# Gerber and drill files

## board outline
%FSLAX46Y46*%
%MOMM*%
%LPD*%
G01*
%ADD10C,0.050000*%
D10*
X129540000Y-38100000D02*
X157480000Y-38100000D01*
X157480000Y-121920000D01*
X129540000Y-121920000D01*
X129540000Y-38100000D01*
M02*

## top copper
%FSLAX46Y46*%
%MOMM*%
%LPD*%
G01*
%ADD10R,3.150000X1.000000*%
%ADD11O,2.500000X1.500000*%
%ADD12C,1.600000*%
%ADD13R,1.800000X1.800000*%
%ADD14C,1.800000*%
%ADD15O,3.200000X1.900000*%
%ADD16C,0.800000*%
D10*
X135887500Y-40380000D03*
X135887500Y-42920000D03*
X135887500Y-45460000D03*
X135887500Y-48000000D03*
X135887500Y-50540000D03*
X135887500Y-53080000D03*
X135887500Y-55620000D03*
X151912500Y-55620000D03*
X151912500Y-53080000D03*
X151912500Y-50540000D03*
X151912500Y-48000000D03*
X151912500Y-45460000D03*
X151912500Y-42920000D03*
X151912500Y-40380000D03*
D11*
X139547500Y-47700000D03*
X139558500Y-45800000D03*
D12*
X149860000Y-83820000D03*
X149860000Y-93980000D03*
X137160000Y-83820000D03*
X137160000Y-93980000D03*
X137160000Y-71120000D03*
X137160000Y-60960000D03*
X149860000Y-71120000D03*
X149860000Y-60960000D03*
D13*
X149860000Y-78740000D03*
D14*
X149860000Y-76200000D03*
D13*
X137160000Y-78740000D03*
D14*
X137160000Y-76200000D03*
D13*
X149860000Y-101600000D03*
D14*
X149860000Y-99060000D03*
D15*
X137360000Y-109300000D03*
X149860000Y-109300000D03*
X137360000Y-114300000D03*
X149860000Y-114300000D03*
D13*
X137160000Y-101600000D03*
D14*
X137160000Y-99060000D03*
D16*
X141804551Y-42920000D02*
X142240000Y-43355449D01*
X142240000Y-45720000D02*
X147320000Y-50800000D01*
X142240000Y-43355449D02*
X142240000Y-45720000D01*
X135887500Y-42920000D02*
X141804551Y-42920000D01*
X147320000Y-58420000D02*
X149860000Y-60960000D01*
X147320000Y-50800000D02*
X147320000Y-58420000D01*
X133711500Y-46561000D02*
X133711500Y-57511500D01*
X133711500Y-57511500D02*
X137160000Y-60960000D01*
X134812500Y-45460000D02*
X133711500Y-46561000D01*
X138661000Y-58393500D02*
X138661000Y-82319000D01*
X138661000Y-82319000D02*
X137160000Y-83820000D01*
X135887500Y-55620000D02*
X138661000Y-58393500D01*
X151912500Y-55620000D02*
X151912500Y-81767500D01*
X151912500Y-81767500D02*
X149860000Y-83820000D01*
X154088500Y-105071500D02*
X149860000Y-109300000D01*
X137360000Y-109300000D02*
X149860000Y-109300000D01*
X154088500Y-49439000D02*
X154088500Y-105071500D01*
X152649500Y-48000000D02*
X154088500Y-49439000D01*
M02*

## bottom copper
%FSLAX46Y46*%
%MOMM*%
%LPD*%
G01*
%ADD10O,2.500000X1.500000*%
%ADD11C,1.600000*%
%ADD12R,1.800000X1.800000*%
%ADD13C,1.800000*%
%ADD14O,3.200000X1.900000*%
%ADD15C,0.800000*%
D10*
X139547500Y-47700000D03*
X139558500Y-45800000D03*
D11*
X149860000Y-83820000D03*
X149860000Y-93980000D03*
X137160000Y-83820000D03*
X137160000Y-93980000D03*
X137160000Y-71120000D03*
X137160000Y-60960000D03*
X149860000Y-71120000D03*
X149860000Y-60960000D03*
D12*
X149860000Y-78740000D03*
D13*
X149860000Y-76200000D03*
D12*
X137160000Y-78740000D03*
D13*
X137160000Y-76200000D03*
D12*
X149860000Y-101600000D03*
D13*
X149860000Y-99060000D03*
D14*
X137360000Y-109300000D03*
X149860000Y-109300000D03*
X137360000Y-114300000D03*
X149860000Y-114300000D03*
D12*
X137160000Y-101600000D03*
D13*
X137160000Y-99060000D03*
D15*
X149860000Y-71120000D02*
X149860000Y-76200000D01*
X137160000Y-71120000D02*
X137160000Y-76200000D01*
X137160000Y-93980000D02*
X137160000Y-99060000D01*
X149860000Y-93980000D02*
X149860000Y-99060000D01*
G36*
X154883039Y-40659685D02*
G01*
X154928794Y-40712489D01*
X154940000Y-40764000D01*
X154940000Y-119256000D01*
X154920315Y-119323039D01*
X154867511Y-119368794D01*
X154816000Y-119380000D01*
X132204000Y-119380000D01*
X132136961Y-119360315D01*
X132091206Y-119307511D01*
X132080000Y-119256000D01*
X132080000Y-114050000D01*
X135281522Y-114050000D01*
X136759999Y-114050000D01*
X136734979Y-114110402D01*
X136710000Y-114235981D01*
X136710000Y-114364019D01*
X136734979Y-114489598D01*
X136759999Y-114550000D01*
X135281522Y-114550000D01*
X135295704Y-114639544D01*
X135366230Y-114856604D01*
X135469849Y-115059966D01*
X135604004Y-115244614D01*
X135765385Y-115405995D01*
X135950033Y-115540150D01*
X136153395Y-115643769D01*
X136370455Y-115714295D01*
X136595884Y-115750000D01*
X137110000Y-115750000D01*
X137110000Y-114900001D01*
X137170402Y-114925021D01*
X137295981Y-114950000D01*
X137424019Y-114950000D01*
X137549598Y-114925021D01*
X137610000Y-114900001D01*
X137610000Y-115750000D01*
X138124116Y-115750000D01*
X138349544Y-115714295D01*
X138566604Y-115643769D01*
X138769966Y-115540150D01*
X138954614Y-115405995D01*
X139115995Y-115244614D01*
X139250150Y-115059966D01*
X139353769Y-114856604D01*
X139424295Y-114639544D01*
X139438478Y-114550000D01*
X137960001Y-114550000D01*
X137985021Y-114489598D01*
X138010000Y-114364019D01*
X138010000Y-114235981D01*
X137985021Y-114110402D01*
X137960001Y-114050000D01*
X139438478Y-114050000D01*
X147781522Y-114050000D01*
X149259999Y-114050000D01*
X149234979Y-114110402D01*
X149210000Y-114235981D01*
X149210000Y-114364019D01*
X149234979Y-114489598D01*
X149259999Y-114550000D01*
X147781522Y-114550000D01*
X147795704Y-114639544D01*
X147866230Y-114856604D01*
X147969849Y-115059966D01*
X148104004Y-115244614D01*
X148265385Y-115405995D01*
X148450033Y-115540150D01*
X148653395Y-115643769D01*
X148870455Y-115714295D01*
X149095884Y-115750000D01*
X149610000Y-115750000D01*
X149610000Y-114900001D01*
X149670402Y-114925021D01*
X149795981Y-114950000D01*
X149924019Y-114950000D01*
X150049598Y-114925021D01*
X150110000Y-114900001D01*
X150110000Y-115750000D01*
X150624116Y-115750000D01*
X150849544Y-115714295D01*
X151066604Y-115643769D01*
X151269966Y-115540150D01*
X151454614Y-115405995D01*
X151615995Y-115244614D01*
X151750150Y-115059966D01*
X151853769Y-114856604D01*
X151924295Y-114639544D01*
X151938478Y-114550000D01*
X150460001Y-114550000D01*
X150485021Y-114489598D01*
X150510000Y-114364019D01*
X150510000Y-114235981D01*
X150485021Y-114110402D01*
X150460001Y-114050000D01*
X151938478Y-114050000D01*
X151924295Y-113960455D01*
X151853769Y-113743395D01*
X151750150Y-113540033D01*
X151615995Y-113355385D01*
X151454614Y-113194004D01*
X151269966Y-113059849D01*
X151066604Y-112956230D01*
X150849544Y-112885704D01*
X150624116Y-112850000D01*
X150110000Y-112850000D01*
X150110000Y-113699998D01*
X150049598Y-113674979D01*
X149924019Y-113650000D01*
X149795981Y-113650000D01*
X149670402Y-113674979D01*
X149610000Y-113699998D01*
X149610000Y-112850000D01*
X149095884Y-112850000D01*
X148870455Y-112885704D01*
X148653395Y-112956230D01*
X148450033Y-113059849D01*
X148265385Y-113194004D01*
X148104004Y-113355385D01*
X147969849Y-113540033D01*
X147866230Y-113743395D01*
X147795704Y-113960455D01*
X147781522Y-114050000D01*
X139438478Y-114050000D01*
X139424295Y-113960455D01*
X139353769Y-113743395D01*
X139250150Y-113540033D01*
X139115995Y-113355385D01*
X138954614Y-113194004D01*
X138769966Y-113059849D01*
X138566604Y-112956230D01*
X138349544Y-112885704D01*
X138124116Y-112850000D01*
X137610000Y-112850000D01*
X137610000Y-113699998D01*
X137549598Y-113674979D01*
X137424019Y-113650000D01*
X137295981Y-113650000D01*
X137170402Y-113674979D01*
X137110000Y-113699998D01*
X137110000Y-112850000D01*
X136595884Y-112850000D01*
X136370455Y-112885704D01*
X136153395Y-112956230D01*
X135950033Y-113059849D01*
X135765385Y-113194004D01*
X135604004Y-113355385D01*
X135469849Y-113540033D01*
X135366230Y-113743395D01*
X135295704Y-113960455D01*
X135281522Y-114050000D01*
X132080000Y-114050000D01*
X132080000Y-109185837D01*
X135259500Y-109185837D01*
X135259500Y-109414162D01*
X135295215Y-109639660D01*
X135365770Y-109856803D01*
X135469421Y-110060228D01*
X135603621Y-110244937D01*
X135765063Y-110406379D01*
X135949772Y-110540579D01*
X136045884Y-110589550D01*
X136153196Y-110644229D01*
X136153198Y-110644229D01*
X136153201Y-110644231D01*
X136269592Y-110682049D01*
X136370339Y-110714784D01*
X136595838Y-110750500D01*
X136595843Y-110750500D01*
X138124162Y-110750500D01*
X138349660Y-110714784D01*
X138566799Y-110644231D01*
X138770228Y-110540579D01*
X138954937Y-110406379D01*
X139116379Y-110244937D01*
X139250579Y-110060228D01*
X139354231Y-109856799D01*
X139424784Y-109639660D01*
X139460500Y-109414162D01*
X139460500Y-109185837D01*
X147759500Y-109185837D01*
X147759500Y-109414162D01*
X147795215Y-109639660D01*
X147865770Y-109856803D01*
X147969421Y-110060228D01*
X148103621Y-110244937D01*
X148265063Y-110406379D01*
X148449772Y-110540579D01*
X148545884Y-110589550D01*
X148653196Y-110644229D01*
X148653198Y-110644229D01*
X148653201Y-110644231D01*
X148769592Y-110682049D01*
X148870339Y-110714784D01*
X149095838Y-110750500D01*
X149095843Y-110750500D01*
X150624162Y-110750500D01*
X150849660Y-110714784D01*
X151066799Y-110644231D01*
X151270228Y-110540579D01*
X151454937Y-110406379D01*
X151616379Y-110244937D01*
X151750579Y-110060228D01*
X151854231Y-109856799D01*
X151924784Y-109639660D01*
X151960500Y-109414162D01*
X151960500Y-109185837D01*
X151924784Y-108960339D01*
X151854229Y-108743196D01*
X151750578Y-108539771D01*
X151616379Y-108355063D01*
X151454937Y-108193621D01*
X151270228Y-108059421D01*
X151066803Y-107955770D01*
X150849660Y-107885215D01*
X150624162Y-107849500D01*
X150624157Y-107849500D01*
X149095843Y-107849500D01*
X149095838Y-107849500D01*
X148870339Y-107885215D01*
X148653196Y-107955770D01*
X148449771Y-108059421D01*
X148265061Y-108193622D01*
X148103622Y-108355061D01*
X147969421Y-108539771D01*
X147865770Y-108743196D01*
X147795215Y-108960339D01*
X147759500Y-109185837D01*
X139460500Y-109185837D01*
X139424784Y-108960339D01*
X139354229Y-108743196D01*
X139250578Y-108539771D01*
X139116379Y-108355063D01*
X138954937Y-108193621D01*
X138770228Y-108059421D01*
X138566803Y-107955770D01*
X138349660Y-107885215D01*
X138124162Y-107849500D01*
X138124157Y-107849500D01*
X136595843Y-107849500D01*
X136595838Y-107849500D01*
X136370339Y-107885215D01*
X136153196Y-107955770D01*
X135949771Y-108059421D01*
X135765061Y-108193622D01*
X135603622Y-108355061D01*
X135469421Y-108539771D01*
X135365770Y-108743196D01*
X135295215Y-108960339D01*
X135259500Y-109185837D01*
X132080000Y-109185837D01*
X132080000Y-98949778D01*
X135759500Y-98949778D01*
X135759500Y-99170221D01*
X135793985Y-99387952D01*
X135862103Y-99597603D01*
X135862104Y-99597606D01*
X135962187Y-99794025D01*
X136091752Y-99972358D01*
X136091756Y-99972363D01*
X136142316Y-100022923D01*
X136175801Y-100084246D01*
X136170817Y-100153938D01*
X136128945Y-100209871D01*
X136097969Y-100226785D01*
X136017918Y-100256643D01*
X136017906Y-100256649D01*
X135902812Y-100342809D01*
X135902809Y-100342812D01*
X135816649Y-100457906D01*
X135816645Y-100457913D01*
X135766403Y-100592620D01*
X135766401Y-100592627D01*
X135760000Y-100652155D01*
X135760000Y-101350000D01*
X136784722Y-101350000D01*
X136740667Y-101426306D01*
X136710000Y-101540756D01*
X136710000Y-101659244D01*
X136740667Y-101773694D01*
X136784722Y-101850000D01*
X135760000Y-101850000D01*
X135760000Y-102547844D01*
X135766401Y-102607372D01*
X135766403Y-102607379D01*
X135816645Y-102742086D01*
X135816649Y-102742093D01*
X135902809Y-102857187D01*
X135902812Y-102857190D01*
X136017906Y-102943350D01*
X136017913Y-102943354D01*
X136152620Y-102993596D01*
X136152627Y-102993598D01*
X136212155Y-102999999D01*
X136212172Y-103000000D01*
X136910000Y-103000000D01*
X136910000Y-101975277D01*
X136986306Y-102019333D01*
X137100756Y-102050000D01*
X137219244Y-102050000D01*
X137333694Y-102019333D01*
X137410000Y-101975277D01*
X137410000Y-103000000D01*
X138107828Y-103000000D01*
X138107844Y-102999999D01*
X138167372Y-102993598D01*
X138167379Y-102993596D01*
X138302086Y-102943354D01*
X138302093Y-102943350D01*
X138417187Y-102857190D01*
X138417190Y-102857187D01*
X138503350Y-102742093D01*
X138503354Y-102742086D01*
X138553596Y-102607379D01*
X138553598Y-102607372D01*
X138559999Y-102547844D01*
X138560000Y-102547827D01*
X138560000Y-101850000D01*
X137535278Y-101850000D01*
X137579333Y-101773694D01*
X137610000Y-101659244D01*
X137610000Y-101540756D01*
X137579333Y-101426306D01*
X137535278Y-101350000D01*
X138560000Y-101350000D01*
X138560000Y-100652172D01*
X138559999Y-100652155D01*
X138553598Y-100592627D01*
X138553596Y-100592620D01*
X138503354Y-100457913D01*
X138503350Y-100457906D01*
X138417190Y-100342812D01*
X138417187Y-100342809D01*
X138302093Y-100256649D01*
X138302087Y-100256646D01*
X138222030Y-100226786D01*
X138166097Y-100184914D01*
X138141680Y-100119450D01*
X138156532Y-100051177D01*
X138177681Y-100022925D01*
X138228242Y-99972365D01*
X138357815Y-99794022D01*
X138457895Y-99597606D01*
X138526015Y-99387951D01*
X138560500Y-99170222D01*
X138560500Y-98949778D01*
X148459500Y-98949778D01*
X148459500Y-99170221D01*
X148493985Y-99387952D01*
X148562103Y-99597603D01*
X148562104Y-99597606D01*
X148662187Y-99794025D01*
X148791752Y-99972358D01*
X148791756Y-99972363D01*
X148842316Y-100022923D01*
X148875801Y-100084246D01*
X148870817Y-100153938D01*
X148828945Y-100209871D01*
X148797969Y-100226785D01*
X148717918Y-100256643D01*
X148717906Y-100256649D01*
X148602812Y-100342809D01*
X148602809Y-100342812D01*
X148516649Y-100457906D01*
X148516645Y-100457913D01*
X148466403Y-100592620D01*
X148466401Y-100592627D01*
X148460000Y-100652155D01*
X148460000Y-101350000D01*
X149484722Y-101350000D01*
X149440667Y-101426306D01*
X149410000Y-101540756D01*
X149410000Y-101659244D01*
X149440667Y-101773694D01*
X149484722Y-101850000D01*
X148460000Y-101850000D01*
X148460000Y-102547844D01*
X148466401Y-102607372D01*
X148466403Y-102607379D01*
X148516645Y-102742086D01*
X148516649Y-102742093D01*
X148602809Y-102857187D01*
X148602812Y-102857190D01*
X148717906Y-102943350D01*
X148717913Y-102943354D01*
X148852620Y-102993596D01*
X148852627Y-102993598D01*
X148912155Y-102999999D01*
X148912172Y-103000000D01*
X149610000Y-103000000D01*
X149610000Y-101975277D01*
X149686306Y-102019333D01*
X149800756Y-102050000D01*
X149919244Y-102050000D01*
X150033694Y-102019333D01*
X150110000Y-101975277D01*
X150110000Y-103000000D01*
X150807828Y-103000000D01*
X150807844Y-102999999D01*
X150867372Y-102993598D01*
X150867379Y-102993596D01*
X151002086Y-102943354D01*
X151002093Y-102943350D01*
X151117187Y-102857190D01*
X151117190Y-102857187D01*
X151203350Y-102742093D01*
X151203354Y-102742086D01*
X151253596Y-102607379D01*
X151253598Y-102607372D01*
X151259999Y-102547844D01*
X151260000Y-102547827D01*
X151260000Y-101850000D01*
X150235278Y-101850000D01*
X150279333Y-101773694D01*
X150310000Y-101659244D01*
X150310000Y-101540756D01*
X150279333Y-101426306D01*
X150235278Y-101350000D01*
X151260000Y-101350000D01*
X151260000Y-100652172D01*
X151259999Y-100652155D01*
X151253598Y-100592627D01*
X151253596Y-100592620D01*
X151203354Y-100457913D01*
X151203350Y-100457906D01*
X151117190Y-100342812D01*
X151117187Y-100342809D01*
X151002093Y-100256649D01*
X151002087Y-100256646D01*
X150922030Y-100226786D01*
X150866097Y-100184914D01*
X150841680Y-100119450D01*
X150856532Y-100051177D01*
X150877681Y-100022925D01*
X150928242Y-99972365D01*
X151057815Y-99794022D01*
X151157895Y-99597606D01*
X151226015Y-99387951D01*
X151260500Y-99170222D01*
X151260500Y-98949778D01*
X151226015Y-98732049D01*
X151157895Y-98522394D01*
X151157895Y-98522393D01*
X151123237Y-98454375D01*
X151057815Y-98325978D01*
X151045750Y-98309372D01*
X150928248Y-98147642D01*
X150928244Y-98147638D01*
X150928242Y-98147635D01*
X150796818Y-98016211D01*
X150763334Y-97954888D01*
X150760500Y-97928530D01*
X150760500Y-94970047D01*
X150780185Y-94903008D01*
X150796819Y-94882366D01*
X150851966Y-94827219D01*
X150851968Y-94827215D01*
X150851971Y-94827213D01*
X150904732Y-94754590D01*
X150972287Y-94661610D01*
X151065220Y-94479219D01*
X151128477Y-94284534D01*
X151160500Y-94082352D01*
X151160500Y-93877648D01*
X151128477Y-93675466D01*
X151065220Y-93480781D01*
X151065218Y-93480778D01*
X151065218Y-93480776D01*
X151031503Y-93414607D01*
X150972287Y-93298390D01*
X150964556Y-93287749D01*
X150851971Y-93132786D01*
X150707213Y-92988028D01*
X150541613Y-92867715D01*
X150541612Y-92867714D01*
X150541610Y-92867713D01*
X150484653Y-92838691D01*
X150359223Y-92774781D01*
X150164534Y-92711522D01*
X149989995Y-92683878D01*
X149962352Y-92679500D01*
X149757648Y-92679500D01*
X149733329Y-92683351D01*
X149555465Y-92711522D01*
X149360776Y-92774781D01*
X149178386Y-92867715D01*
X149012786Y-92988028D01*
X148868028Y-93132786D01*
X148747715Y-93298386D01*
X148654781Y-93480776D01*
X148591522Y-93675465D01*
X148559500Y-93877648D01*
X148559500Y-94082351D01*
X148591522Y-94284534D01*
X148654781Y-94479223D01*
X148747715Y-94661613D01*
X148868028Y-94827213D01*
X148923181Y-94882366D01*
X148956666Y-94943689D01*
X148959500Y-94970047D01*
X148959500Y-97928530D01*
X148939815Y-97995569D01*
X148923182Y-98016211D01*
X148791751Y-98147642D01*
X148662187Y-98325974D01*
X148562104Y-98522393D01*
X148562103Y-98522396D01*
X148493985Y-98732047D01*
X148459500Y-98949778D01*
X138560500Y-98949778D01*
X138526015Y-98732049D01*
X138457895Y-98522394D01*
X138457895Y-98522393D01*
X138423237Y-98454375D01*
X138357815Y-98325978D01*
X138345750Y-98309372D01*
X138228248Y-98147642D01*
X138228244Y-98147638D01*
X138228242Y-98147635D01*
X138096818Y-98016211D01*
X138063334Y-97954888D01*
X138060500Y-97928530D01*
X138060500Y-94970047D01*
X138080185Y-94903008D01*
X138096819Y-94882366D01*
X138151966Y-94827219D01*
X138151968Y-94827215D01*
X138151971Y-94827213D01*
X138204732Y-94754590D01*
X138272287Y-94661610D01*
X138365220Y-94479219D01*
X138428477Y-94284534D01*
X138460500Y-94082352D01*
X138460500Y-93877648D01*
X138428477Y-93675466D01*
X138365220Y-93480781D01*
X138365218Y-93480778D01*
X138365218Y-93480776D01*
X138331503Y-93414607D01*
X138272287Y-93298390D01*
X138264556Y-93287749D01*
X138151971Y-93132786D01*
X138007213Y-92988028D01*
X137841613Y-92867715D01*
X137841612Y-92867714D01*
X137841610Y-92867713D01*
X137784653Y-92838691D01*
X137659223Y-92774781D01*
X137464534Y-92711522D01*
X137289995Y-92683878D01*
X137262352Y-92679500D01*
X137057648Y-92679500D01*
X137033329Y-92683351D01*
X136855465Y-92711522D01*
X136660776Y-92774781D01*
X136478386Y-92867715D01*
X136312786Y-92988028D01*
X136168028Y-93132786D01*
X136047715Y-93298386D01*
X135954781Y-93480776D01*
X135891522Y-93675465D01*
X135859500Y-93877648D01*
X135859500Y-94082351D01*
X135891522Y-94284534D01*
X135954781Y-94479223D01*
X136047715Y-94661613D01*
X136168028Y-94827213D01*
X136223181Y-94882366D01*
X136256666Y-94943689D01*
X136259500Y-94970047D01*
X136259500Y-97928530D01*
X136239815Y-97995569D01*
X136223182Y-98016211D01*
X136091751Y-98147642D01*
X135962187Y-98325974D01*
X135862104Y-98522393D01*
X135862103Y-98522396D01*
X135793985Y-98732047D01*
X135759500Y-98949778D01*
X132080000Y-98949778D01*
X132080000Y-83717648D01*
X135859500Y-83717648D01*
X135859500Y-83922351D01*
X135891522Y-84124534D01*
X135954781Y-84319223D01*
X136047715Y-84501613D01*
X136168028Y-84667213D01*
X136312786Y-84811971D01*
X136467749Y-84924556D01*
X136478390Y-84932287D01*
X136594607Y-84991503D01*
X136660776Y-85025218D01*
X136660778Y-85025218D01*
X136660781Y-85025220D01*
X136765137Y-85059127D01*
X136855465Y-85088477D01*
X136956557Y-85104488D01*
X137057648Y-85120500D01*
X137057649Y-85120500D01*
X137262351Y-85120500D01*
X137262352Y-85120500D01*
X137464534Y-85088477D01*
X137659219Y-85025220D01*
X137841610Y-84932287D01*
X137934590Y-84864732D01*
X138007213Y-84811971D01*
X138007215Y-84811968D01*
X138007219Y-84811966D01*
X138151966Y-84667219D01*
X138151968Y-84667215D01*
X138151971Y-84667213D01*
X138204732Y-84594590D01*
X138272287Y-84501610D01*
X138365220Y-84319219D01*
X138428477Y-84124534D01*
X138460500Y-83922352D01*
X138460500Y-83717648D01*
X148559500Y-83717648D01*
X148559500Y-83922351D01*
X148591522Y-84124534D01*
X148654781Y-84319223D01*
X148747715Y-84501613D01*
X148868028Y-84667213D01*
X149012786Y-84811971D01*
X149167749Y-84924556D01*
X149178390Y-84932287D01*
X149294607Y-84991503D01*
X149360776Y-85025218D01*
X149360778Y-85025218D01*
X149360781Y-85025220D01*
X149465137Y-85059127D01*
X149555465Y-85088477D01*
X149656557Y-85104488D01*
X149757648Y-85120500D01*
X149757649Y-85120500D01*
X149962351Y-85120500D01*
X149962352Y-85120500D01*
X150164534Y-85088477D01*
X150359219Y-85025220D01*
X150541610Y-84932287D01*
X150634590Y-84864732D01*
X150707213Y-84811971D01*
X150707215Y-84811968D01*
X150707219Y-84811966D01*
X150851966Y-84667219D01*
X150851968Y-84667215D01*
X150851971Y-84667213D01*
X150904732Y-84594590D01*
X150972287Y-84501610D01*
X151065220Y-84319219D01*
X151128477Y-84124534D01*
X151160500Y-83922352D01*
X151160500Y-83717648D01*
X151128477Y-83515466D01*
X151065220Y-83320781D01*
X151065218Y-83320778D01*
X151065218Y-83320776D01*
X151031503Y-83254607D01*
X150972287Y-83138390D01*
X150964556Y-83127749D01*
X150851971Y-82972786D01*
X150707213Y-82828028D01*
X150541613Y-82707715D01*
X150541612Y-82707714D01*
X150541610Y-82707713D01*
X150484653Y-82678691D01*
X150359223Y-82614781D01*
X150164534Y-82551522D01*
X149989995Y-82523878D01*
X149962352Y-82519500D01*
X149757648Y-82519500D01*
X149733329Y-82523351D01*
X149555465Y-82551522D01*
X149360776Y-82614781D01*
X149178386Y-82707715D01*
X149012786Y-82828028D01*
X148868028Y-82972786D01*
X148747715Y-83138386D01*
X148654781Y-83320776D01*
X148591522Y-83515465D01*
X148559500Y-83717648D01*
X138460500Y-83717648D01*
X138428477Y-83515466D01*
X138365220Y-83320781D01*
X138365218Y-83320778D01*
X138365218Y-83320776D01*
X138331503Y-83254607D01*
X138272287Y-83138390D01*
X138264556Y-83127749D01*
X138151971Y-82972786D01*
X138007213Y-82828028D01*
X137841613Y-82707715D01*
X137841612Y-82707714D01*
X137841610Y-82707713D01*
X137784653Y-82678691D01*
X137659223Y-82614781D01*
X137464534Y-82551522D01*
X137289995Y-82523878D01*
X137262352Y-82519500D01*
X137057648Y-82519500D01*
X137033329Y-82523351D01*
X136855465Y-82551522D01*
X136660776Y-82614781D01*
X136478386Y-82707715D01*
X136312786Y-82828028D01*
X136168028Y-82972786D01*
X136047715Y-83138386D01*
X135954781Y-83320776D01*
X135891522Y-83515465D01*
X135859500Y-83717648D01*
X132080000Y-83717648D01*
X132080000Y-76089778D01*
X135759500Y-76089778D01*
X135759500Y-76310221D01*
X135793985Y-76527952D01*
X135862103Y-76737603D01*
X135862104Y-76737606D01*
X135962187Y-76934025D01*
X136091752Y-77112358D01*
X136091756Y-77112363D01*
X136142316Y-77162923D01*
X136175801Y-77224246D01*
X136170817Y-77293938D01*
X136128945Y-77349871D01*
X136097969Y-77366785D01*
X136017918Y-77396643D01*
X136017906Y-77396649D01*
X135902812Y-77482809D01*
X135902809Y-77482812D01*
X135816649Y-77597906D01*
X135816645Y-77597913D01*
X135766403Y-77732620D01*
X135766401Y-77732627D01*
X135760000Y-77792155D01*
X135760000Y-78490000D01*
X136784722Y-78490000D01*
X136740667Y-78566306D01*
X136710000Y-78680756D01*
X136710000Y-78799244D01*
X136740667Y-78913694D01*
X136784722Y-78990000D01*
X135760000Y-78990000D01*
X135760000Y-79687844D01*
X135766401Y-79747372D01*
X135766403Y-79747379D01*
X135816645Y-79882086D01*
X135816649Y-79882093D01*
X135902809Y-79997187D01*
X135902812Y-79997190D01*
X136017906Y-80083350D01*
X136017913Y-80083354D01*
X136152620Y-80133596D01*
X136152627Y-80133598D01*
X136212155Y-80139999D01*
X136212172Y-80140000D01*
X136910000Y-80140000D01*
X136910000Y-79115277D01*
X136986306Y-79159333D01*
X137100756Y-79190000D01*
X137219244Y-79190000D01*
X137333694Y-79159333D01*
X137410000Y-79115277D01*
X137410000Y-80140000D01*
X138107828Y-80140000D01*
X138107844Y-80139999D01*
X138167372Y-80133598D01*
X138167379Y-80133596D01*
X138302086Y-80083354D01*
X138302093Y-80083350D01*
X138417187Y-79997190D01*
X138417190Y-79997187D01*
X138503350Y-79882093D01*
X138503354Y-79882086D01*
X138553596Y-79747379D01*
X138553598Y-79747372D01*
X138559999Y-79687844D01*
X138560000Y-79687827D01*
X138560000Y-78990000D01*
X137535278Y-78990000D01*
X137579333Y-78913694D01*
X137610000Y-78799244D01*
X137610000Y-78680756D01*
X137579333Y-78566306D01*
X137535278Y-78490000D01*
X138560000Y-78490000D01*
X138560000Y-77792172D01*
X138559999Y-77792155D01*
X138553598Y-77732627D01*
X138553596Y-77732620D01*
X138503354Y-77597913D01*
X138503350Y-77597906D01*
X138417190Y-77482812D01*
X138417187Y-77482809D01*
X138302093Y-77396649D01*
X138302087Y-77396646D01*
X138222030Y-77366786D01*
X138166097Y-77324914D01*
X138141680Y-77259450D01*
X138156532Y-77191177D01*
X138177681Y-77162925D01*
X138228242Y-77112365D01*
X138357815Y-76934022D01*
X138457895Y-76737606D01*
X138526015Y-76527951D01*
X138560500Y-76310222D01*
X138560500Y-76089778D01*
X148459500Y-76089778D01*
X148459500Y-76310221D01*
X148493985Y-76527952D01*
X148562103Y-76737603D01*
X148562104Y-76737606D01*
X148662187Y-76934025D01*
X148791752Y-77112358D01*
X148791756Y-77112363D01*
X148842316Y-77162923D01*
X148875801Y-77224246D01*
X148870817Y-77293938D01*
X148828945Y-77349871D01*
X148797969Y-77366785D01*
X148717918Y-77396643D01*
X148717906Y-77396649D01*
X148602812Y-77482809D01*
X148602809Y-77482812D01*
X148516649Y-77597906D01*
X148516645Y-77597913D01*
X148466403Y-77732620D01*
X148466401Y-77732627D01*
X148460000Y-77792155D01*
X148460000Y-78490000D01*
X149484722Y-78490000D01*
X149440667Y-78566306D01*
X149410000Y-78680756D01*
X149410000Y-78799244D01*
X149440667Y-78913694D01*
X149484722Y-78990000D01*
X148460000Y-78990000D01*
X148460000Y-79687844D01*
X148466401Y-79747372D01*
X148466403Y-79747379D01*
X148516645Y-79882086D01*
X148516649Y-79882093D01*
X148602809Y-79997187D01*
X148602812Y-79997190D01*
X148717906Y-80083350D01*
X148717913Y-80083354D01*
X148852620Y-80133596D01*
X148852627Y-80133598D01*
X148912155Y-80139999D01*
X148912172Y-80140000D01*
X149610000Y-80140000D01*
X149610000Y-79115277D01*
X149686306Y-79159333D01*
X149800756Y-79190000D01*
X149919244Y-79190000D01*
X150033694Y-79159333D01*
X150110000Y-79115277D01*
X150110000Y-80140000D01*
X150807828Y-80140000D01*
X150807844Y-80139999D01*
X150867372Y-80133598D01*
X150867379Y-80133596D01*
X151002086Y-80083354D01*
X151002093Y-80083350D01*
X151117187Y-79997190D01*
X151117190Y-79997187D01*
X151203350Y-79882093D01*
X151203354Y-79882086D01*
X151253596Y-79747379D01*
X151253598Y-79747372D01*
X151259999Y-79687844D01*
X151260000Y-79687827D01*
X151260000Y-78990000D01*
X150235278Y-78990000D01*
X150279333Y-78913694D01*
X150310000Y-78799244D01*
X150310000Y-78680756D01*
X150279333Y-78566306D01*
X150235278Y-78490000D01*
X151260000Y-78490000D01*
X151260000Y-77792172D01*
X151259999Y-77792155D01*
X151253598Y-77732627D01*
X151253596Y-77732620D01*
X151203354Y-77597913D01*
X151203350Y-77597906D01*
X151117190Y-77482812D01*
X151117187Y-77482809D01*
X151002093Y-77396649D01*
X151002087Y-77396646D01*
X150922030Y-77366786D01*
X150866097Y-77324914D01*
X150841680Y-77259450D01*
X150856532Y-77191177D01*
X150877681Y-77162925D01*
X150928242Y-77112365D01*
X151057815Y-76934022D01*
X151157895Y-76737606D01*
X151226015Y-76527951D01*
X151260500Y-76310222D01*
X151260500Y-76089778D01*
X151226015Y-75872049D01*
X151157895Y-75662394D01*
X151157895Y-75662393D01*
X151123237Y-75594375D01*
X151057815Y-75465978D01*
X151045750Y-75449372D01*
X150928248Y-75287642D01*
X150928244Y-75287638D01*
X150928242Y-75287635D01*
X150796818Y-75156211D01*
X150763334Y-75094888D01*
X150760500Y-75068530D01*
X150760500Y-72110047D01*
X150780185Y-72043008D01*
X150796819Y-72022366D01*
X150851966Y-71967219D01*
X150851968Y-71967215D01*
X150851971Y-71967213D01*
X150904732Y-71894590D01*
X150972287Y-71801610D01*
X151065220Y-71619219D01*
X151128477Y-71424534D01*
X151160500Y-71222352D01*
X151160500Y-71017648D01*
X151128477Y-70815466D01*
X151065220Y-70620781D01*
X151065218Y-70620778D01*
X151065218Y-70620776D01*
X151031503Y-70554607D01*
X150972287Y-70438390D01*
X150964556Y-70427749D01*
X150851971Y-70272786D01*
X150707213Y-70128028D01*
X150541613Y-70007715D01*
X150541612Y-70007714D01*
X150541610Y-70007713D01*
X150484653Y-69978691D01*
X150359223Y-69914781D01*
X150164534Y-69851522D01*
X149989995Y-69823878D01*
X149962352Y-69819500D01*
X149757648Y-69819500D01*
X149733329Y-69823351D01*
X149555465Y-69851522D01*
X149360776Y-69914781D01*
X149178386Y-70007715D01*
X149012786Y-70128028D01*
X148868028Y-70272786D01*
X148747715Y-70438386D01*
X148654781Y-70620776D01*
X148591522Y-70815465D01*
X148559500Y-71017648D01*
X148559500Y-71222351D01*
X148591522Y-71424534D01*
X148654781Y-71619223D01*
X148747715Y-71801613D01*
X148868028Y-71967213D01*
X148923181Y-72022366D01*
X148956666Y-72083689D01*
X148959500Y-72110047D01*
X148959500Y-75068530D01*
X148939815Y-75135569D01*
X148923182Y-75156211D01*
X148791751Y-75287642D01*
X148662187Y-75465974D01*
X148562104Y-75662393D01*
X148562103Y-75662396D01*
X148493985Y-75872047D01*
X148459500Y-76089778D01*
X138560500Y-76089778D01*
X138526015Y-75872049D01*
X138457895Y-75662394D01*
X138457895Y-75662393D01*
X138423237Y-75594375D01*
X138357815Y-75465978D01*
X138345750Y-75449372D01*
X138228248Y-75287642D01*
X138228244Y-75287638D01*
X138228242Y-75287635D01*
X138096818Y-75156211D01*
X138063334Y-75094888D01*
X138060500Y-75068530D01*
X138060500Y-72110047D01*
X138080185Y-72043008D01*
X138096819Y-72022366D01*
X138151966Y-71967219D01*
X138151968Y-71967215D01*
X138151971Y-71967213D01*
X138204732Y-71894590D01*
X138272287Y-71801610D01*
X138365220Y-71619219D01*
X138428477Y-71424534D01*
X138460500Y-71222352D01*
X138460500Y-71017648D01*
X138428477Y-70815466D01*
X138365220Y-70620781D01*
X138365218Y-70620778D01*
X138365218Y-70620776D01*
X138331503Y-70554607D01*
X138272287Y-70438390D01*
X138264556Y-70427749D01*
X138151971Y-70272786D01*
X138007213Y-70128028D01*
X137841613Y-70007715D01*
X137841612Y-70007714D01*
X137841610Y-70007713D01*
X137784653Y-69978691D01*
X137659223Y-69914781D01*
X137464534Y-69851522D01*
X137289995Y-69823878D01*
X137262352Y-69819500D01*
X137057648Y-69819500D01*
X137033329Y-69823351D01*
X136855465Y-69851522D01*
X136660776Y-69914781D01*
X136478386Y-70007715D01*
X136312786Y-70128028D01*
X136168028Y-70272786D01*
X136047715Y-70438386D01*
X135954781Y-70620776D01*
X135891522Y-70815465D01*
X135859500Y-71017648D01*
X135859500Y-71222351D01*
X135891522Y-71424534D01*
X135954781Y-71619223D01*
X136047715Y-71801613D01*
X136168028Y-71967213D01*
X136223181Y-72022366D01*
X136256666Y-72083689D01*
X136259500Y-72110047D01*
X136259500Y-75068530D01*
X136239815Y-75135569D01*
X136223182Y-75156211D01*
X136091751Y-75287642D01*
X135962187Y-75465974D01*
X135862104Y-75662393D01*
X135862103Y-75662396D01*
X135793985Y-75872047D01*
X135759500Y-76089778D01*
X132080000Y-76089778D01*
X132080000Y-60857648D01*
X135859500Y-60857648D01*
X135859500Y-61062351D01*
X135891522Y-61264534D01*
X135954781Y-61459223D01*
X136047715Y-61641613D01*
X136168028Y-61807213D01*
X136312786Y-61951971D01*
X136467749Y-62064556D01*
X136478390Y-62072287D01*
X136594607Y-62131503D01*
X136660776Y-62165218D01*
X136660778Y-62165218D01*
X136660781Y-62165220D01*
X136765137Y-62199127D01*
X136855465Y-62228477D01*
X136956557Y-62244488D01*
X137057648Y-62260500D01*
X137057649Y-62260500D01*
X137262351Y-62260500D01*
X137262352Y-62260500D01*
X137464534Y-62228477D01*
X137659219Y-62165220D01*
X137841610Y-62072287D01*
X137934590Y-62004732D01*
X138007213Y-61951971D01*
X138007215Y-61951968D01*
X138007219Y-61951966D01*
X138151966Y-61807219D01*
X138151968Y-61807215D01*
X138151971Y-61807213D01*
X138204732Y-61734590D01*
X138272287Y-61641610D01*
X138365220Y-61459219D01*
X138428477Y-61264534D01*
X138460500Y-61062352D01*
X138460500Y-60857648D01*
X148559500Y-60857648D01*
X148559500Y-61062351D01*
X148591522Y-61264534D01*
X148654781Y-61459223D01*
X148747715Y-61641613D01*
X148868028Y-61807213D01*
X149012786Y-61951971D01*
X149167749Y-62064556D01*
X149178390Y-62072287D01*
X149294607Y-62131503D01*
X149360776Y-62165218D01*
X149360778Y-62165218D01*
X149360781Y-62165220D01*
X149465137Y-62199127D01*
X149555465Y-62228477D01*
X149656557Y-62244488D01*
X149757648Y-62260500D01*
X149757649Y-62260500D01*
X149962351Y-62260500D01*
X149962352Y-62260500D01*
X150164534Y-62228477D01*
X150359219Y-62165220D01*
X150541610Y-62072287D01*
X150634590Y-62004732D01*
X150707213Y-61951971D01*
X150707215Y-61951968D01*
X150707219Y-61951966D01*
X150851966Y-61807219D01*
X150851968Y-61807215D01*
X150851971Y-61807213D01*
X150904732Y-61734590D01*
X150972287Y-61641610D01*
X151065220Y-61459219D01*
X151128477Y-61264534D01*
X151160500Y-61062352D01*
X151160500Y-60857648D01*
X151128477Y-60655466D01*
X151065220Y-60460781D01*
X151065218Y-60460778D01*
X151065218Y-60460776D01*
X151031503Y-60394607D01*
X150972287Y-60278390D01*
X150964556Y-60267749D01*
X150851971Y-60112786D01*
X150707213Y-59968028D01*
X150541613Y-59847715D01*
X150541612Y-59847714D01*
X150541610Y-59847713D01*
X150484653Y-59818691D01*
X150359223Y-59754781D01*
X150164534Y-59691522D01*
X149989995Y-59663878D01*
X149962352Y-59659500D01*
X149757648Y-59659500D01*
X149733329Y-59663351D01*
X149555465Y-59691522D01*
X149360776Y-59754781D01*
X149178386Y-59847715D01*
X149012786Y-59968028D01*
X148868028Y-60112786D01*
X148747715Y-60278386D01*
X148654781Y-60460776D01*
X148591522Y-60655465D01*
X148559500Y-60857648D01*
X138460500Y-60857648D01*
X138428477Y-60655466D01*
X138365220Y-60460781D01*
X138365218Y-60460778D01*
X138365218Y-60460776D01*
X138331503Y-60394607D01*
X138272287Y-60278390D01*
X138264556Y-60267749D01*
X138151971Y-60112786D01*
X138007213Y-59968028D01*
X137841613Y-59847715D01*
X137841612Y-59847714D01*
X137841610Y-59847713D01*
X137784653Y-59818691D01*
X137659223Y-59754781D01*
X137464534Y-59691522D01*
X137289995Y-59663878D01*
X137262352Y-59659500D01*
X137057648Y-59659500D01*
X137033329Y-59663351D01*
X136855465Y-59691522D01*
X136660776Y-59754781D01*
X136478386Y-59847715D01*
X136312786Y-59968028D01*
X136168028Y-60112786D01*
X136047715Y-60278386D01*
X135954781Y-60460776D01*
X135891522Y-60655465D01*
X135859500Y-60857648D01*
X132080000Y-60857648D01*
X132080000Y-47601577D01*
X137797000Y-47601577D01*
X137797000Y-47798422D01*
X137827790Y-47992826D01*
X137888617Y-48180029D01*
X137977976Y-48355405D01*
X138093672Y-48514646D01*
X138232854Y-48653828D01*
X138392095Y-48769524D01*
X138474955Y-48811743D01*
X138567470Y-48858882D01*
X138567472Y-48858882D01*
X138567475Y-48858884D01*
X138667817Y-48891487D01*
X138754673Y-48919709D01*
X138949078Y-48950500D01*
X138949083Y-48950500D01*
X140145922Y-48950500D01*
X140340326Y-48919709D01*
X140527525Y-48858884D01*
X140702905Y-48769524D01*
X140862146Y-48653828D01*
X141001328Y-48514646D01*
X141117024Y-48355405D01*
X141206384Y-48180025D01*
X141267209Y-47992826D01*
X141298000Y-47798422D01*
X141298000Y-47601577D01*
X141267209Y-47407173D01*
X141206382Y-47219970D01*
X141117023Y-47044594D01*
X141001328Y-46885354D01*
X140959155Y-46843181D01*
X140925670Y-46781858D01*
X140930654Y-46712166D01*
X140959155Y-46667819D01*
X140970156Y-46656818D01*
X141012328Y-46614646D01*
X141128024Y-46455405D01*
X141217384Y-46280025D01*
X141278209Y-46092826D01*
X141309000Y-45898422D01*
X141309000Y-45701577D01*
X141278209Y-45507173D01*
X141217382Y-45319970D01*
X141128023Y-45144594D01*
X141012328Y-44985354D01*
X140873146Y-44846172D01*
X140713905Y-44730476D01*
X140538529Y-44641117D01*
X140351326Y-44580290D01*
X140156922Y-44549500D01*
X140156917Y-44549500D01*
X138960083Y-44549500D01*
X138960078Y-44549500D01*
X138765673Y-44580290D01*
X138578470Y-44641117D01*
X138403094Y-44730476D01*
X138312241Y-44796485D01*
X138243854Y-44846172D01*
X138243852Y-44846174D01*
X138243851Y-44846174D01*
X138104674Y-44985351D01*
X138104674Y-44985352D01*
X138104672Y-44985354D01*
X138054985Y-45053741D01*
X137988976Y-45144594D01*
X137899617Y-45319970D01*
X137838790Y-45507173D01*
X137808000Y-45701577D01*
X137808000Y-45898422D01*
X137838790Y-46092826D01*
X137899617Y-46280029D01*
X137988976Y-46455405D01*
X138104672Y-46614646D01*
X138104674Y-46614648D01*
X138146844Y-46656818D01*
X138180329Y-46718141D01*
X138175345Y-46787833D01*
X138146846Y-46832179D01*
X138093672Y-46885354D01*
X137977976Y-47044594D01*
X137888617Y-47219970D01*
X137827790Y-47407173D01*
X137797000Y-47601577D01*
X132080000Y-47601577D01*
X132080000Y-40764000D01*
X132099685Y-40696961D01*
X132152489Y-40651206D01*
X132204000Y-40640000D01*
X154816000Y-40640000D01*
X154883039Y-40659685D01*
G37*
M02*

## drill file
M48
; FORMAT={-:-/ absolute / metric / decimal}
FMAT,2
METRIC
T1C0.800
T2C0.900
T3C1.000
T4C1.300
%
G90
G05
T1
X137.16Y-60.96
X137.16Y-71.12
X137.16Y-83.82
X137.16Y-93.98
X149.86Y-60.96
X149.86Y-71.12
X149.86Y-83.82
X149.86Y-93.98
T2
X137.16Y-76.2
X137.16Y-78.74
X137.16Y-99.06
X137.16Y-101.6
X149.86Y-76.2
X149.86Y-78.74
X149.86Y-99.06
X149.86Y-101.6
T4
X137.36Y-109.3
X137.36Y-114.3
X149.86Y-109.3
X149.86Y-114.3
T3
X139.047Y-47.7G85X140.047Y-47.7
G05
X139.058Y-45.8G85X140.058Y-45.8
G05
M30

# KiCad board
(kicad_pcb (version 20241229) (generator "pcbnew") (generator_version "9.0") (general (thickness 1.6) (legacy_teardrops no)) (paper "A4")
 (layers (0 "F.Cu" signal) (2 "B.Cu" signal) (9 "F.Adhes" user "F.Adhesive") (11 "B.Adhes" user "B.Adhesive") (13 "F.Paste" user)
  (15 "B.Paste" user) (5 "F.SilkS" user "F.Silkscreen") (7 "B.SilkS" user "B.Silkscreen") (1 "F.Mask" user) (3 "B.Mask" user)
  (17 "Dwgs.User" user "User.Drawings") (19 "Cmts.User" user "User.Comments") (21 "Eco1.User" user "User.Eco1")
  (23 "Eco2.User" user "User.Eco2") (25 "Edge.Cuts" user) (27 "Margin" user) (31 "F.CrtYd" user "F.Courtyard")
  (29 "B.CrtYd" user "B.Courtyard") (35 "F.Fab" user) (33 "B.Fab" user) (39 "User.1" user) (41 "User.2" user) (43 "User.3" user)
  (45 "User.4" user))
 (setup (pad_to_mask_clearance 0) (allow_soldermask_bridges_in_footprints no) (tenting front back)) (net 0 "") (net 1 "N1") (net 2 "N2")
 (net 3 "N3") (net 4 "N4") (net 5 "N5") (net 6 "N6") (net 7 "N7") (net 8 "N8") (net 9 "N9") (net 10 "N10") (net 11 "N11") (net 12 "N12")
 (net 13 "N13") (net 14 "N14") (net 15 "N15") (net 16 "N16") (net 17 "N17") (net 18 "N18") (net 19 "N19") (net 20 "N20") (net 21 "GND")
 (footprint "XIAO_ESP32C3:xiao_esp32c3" (layer "F.Cu") (at 144.4875 49.8)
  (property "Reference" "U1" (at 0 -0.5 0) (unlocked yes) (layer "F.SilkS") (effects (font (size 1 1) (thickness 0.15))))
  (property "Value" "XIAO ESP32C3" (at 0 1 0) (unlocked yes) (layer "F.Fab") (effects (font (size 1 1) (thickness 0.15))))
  (pad "1" smd rect (at -8.6 -9.42) (size 3.15 1) (layers "F.Cu" "F.Mask" "F.Paste") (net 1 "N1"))
  (pad "2" smd rect (at -8.6 -6.88) (size 3.15 1) (layers "F.Cu" "F.Mask" "F.Paste") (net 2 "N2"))
  (pad "3" smd rect (at -8.6 -4.34) (size 3.15 1) (layers "F.Cu" "F.Mask" "F.Paste") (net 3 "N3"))
  (pad "4" smd rect (at -8.6 -1.8) (size 3.15 1) (layers "F.Cu" "F.Mask" "F.Paste") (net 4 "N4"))
  (pad "5" smd rect (at -8.6 0.74) (size 3.15 1) (layers "F.Cu" "F.Mask" "F.Paste") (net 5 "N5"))
  (pad "6" smd rect (at -8.6 3.28) (size 3.15 1) (layers "F.Cu" "F.Mask" "F.Paste") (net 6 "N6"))
  (pad "7" smd rect (at -8.6 5.82) (size 3.15 1) (layers "F.Cu" "F.Mask" "F.Paste") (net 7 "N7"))
  (pad "8" smd rect (at 7.425 5.82) (size 3.15 1) (layers "F.Cu" "F.Mask" "F.Paste") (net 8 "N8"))
  (pad "9" smd rect (at 7.425 3.28) (size 3.15 1) (layers "F.Cu" "F.Mask" "F.Paste") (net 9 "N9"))
  (pad "10" smd rect (at 7.425 0.74) (size 3.15 1) (layers "F.Cu" "F.Mask" "F.Paste") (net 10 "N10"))
  (pad "11" smd rect (at 7.425 -1.8) (size 3.15 1) (layers "F.Cu" "F.Mask" "F.Paste") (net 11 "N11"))
  (pad "12" smd rect (at 7.425 -4.34) (size 3.15 1) (layers "F.Cu" "F.Mask" "F.Paste") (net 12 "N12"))
  (pad "13" smd rect (at 7.425 -6.88) (size 3.15 1) (layers "F.Cu" "F.Mask" "F.Paste") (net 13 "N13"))
  (pad "14" smd rect (at 7.425 -9.42) (size 3.15 1) (layers "F.Cu" "F.Mask" "F.Paste") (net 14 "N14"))
  (pad "B+" thru_hole oval (at -4.94 -2.1) (size 2.5 1.5) (drill oval 2 1) (layers "*.Cu" "*.Mask") (remove_unused_layers no) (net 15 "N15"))
  (pad "B-" thru_hole oval (at -4.929 -4) (size 2.5 1.5) (drill oval 2 1) (layers "*.Cu" "*.Mask") (remove_unused_layers no) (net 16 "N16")))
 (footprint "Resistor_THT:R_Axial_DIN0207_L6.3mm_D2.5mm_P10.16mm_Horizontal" (layer "F.Cu") (at 149.86 83.82 -90)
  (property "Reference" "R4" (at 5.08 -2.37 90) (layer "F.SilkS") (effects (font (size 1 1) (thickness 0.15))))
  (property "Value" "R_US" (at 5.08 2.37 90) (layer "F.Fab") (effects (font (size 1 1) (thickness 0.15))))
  (pad "1" thru_hole circle (at 0 0 270) (size 1.6 1.6) (drill 0.8) (layers "*.Cu" "*.Mask") (remove_unused_layers no) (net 8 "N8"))
  (pad "2" thru_hole circle (at 10.16 0 270) (size 1.6 1.6) (drill 0.8) (layers "*.Cu" "*.Mask") (remove_unused_layers no) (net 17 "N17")))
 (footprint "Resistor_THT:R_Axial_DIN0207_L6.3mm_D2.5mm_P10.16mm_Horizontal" (layer "F.Cu") (at 137.16 83.82 -90)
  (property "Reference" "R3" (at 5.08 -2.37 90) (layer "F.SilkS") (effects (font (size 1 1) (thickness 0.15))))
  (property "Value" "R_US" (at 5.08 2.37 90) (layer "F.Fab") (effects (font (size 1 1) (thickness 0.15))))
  (pad "1" thru_hole circle (at 0 0 270) (size 1.6 1.6) (drill 0.8) (layers "*.Cu" "*.Mask") (remove_unused_layers no) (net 7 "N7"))
  (pad "2" thru_hole circle (at 10.16 0 270) (size 1.6 1.6) (drill 0.8) (layers "*.Cu" "*.Mask") (remove_unused_layers no) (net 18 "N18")))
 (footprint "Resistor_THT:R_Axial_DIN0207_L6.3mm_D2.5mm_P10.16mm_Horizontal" (layer "F.Cu") (at 137.16 71.12 90)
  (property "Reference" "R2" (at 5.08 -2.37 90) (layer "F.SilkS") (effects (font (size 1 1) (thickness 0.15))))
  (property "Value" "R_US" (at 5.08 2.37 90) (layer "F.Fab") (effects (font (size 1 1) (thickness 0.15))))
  (pad "1" thru_hole circle (at 0 0 90) (size 1.6 1.6) (drill 0.8) (layers "*.Cu" "*.Mask") (remove_unused_layers no) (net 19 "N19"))
  (pad "2" thru_hole circle (at 10.16 0 90) (size 1.6 1.6) (drill 0.8) (layers "*.Cu" "*.Mask") (remove_unused_layers no) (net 3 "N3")))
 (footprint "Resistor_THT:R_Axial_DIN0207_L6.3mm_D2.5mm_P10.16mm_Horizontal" (layer "F.Cu") (at 149.86 71.12 90)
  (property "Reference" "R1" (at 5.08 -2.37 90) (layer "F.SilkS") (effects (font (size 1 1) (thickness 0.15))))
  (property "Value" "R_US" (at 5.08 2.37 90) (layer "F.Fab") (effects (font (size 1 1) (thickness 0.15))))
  (pad "1" thru_hole circle (at 0 0 90) (size 1.6 1.6) (drill 0.8) (layers "*.Cu" "*.Mask") (remove_unused_layers no) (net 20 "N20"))
  (pad "2" thru_hole circle (at 10.16 0 90) (size 1.6 1.6) (drill 0.8) (layers "*.Cu" "*.Mask") (remove_unused_layers no) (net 2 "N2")))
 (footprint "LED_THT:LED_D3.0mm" (layer "F.Cu") (at 149.86 78.74 90)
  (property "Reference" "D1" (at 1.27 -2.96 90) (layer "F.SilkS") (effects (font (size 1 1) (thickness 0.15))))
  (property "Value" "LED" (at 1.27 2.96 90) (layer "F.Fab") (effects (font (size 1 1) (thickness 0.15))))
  (pad "1" thru_hole rect (at 0 0 90) (size 1.8 1.8) (drill 0.9) (layers "*.Cu" "*.Mask") (remove_unused_layers no) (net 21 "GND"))
  (pad "2" thru_hole circle (at 2.54 0 90) (size 1.8 1.8) (drill 0.9) (layers "*.Cu" "*.Mask") (remove_unused_layers no) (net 20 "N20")))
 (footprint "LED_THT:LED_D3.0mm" (layer "F.Cu") (at 137.16 78.74 90)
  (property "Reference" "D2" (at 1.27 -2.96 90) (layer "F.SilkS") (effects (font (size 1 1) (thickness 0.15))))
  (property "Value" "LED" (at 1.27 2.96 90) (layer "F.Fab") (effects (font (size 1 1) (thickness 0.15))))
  (pad "1" thru_hole rect (at 0 0 90) (size 1.8 1.8) (drill 0.9) (layers "*.Cu" "*.Mask") (remove_unused_layers no) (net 21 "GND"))
  (pad "2" thru_hole circle (at 2.54 0 90) (size 1.8 1.8) (drill 0.9) (layers "*.Cu" "*.Mask") (remove_unused_layers no) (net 19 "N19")))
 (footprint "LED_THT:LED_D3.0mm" (layer "F.Cu") (at 149.86 101.6 90)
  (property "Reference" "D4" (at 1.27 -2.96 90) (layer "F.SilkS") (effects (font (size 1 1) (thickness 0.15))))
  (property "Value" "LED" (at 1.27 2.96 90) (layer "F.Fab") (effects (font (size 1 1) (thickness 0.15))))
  (pad "1" thru_hole rect (at 0 0 90) (size 1.8 1.8) (drill 0.9) (layers "*.Cu" "*.Mask") (remove_unused_layers no) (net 21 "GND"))
  (pad "2" thru_hole circle (at 2.54 0 90) (size 1.8 1.8) (drill 0.9) (layers "*.Cu" "*.Mask") (remove_unused_layers no) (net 17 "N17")))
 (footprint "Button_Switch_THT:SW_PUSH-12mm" (layer "F.Cu") (at 137.36 109.3)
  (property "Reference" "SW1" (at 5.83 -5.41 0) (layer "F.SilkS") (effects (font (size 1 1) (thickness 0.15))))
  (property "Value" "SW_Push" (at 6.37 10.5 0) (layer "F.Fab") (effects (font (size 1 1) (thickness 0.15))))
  (pad "1" thru_hole oval (at 0 0) (size 3.2 1.9) (drill 1.3) (layers "*.Cu" "*.Mask") (remove_unused_layers no) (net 11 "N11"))
  (pad "1" thru_hole oval (at 12.5 0) (size 3.2 1.9) (drill 1.3) (layers "*.Cu" "*.Mask") (remove_unused_layers no) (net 11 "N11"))
  (pad "2" thru_hole oval (at 0 5) (size 3.2 1.9) (drill 1.3) (layers "*.Cu" "*.Mask") (remove_unused_layers no) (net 21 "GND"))
  (pad "2" thru_hole oval (at 12.5 5) (size 3.2 1.9) (drill 1.3) (layers "*.Cu" "*.Mask") (remove_unused_layers no) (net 21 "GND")))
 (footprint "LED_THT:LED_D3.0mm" (layer "F.Cu") (at 137.16 101.6 90)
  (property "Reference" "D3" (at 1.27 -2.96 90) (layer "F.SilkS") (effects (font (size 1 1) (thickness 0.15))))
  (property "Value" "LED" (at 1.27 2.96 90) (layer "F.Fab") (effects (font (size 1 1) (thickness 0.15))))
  (pad "1" thru_hole rect (at 0 0 90) (size 1.8 1.8) (drill 0.9) (layers "*.Cu" "*.Mask") (remove_unused_layers no) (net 21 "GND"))
  (pad "2" thru_hole circle (at 2.54 0 90) (size 1.8 1.8) (drill 0.9) (layers "*.Cu" "*.Mask") (remove_unused_layers no) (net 18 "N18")))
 (gr_rect (start 129.54 38.1) (end 157.48 121.92) (stroke (width 0.05) (type default)) (fill no) (layer "Edge.Cuts"))
 (segment (start 149.86 71.12) (end 149.86 76.2) (width 0.8) (layer "B.Cu") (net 20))
 (segment (start 137.16 71.12) (end 137.16 76.2) (width 0.8) (layer "B.Cu") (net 19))
 (segment (start 137.16 93.98) (end 137.16 99.06) (width 0.8) (layer "B.Cu") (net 18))
 (segment (start 149.86 93.98) (end 149.86 99.06) (width 0.8) (layer "B.Cu") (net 17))
 (segment (start 141.804551 42.92) (end 142.24 43.355449) (width 0.8) (layer "F.Cu") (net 2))
 (segment (start 142.24 45.72) (end 147.32 50.8) (width 0.8) (layer "F.Cu") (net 2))
 (segment (start 142.24 43.355449) (end 142.24 45.72) (width 0.8) (layer "F.Cu") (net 2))
 (segment (start 135.8875 42.92) (end 141.804551 42.92) (width 0.8) (layer "F.Cu") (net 2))
 (segment (start 147.32 58.42) (end 149.86 60.96) (width 0.8) (layer "F.Cu") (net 2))
 (segment (start 147.32 50.8) (end 147.32 58.42) (width 0.8) (layer "F.Cu") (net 2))
 (segment (start 133.7115 46.561) (end 133.7115 57.5115) (width 0.8) (layer "F.Cu") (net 3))
 (segment (start 133.7115 57.5115) (end 137.16 60.96) (width 0.8) (layer "F.Cu") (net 3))
 (segment (start 134.8125 45.46) (end 133.7115 46.561) (width 0.8) (layer "F.Cu") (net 3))
 (segment (start 138.661 58.3935) (end 138.661 82.319) (width 0.8) (layer "F.Cu") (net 7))
 (segment (start 138.661 82.319) (end 137.16 83.82) (width 0.8) (layer "F.Cu") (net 7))
 (segment (start 135.8875 55.62) (end 138.661 58.3935) (width 0.8) (layer "F.Cu") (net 7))
 (segment (start 151.9125 55.62) (end 151.9125 81.7675) (width 0.8) (layer "F.Cu") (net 8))
 (segment (start 151.9125 81.7675) (end 149.86 83.82) (width 0.8) (layer "F.Cu") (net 8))
 (segment (start 154.0885 105.0715) (end 149.86 109.3) (width 0.8) (layer "F.Cu") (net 11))
 (segment (start 137.36 109.3) (end 149.86 109.3) (width 0.8) (layer "F.Cu") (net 11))
 (segment (start 154.0885 49.439) (end 154.0885 105.0715) (width 0.8) (layer "F.Cu") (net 11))
 (segment (start 152.6495 48) (end 154.0885 49.439) (width 0.8) (layer "F.Cu") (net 11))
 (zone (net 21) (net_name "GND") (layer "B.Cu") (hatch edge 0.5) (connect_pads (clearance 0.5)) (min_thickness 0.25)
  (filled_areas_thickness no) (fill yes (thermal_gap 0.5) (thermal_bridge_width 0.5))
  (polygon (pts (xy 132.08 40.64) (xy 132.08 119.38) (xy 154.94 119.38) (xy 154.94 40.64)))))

